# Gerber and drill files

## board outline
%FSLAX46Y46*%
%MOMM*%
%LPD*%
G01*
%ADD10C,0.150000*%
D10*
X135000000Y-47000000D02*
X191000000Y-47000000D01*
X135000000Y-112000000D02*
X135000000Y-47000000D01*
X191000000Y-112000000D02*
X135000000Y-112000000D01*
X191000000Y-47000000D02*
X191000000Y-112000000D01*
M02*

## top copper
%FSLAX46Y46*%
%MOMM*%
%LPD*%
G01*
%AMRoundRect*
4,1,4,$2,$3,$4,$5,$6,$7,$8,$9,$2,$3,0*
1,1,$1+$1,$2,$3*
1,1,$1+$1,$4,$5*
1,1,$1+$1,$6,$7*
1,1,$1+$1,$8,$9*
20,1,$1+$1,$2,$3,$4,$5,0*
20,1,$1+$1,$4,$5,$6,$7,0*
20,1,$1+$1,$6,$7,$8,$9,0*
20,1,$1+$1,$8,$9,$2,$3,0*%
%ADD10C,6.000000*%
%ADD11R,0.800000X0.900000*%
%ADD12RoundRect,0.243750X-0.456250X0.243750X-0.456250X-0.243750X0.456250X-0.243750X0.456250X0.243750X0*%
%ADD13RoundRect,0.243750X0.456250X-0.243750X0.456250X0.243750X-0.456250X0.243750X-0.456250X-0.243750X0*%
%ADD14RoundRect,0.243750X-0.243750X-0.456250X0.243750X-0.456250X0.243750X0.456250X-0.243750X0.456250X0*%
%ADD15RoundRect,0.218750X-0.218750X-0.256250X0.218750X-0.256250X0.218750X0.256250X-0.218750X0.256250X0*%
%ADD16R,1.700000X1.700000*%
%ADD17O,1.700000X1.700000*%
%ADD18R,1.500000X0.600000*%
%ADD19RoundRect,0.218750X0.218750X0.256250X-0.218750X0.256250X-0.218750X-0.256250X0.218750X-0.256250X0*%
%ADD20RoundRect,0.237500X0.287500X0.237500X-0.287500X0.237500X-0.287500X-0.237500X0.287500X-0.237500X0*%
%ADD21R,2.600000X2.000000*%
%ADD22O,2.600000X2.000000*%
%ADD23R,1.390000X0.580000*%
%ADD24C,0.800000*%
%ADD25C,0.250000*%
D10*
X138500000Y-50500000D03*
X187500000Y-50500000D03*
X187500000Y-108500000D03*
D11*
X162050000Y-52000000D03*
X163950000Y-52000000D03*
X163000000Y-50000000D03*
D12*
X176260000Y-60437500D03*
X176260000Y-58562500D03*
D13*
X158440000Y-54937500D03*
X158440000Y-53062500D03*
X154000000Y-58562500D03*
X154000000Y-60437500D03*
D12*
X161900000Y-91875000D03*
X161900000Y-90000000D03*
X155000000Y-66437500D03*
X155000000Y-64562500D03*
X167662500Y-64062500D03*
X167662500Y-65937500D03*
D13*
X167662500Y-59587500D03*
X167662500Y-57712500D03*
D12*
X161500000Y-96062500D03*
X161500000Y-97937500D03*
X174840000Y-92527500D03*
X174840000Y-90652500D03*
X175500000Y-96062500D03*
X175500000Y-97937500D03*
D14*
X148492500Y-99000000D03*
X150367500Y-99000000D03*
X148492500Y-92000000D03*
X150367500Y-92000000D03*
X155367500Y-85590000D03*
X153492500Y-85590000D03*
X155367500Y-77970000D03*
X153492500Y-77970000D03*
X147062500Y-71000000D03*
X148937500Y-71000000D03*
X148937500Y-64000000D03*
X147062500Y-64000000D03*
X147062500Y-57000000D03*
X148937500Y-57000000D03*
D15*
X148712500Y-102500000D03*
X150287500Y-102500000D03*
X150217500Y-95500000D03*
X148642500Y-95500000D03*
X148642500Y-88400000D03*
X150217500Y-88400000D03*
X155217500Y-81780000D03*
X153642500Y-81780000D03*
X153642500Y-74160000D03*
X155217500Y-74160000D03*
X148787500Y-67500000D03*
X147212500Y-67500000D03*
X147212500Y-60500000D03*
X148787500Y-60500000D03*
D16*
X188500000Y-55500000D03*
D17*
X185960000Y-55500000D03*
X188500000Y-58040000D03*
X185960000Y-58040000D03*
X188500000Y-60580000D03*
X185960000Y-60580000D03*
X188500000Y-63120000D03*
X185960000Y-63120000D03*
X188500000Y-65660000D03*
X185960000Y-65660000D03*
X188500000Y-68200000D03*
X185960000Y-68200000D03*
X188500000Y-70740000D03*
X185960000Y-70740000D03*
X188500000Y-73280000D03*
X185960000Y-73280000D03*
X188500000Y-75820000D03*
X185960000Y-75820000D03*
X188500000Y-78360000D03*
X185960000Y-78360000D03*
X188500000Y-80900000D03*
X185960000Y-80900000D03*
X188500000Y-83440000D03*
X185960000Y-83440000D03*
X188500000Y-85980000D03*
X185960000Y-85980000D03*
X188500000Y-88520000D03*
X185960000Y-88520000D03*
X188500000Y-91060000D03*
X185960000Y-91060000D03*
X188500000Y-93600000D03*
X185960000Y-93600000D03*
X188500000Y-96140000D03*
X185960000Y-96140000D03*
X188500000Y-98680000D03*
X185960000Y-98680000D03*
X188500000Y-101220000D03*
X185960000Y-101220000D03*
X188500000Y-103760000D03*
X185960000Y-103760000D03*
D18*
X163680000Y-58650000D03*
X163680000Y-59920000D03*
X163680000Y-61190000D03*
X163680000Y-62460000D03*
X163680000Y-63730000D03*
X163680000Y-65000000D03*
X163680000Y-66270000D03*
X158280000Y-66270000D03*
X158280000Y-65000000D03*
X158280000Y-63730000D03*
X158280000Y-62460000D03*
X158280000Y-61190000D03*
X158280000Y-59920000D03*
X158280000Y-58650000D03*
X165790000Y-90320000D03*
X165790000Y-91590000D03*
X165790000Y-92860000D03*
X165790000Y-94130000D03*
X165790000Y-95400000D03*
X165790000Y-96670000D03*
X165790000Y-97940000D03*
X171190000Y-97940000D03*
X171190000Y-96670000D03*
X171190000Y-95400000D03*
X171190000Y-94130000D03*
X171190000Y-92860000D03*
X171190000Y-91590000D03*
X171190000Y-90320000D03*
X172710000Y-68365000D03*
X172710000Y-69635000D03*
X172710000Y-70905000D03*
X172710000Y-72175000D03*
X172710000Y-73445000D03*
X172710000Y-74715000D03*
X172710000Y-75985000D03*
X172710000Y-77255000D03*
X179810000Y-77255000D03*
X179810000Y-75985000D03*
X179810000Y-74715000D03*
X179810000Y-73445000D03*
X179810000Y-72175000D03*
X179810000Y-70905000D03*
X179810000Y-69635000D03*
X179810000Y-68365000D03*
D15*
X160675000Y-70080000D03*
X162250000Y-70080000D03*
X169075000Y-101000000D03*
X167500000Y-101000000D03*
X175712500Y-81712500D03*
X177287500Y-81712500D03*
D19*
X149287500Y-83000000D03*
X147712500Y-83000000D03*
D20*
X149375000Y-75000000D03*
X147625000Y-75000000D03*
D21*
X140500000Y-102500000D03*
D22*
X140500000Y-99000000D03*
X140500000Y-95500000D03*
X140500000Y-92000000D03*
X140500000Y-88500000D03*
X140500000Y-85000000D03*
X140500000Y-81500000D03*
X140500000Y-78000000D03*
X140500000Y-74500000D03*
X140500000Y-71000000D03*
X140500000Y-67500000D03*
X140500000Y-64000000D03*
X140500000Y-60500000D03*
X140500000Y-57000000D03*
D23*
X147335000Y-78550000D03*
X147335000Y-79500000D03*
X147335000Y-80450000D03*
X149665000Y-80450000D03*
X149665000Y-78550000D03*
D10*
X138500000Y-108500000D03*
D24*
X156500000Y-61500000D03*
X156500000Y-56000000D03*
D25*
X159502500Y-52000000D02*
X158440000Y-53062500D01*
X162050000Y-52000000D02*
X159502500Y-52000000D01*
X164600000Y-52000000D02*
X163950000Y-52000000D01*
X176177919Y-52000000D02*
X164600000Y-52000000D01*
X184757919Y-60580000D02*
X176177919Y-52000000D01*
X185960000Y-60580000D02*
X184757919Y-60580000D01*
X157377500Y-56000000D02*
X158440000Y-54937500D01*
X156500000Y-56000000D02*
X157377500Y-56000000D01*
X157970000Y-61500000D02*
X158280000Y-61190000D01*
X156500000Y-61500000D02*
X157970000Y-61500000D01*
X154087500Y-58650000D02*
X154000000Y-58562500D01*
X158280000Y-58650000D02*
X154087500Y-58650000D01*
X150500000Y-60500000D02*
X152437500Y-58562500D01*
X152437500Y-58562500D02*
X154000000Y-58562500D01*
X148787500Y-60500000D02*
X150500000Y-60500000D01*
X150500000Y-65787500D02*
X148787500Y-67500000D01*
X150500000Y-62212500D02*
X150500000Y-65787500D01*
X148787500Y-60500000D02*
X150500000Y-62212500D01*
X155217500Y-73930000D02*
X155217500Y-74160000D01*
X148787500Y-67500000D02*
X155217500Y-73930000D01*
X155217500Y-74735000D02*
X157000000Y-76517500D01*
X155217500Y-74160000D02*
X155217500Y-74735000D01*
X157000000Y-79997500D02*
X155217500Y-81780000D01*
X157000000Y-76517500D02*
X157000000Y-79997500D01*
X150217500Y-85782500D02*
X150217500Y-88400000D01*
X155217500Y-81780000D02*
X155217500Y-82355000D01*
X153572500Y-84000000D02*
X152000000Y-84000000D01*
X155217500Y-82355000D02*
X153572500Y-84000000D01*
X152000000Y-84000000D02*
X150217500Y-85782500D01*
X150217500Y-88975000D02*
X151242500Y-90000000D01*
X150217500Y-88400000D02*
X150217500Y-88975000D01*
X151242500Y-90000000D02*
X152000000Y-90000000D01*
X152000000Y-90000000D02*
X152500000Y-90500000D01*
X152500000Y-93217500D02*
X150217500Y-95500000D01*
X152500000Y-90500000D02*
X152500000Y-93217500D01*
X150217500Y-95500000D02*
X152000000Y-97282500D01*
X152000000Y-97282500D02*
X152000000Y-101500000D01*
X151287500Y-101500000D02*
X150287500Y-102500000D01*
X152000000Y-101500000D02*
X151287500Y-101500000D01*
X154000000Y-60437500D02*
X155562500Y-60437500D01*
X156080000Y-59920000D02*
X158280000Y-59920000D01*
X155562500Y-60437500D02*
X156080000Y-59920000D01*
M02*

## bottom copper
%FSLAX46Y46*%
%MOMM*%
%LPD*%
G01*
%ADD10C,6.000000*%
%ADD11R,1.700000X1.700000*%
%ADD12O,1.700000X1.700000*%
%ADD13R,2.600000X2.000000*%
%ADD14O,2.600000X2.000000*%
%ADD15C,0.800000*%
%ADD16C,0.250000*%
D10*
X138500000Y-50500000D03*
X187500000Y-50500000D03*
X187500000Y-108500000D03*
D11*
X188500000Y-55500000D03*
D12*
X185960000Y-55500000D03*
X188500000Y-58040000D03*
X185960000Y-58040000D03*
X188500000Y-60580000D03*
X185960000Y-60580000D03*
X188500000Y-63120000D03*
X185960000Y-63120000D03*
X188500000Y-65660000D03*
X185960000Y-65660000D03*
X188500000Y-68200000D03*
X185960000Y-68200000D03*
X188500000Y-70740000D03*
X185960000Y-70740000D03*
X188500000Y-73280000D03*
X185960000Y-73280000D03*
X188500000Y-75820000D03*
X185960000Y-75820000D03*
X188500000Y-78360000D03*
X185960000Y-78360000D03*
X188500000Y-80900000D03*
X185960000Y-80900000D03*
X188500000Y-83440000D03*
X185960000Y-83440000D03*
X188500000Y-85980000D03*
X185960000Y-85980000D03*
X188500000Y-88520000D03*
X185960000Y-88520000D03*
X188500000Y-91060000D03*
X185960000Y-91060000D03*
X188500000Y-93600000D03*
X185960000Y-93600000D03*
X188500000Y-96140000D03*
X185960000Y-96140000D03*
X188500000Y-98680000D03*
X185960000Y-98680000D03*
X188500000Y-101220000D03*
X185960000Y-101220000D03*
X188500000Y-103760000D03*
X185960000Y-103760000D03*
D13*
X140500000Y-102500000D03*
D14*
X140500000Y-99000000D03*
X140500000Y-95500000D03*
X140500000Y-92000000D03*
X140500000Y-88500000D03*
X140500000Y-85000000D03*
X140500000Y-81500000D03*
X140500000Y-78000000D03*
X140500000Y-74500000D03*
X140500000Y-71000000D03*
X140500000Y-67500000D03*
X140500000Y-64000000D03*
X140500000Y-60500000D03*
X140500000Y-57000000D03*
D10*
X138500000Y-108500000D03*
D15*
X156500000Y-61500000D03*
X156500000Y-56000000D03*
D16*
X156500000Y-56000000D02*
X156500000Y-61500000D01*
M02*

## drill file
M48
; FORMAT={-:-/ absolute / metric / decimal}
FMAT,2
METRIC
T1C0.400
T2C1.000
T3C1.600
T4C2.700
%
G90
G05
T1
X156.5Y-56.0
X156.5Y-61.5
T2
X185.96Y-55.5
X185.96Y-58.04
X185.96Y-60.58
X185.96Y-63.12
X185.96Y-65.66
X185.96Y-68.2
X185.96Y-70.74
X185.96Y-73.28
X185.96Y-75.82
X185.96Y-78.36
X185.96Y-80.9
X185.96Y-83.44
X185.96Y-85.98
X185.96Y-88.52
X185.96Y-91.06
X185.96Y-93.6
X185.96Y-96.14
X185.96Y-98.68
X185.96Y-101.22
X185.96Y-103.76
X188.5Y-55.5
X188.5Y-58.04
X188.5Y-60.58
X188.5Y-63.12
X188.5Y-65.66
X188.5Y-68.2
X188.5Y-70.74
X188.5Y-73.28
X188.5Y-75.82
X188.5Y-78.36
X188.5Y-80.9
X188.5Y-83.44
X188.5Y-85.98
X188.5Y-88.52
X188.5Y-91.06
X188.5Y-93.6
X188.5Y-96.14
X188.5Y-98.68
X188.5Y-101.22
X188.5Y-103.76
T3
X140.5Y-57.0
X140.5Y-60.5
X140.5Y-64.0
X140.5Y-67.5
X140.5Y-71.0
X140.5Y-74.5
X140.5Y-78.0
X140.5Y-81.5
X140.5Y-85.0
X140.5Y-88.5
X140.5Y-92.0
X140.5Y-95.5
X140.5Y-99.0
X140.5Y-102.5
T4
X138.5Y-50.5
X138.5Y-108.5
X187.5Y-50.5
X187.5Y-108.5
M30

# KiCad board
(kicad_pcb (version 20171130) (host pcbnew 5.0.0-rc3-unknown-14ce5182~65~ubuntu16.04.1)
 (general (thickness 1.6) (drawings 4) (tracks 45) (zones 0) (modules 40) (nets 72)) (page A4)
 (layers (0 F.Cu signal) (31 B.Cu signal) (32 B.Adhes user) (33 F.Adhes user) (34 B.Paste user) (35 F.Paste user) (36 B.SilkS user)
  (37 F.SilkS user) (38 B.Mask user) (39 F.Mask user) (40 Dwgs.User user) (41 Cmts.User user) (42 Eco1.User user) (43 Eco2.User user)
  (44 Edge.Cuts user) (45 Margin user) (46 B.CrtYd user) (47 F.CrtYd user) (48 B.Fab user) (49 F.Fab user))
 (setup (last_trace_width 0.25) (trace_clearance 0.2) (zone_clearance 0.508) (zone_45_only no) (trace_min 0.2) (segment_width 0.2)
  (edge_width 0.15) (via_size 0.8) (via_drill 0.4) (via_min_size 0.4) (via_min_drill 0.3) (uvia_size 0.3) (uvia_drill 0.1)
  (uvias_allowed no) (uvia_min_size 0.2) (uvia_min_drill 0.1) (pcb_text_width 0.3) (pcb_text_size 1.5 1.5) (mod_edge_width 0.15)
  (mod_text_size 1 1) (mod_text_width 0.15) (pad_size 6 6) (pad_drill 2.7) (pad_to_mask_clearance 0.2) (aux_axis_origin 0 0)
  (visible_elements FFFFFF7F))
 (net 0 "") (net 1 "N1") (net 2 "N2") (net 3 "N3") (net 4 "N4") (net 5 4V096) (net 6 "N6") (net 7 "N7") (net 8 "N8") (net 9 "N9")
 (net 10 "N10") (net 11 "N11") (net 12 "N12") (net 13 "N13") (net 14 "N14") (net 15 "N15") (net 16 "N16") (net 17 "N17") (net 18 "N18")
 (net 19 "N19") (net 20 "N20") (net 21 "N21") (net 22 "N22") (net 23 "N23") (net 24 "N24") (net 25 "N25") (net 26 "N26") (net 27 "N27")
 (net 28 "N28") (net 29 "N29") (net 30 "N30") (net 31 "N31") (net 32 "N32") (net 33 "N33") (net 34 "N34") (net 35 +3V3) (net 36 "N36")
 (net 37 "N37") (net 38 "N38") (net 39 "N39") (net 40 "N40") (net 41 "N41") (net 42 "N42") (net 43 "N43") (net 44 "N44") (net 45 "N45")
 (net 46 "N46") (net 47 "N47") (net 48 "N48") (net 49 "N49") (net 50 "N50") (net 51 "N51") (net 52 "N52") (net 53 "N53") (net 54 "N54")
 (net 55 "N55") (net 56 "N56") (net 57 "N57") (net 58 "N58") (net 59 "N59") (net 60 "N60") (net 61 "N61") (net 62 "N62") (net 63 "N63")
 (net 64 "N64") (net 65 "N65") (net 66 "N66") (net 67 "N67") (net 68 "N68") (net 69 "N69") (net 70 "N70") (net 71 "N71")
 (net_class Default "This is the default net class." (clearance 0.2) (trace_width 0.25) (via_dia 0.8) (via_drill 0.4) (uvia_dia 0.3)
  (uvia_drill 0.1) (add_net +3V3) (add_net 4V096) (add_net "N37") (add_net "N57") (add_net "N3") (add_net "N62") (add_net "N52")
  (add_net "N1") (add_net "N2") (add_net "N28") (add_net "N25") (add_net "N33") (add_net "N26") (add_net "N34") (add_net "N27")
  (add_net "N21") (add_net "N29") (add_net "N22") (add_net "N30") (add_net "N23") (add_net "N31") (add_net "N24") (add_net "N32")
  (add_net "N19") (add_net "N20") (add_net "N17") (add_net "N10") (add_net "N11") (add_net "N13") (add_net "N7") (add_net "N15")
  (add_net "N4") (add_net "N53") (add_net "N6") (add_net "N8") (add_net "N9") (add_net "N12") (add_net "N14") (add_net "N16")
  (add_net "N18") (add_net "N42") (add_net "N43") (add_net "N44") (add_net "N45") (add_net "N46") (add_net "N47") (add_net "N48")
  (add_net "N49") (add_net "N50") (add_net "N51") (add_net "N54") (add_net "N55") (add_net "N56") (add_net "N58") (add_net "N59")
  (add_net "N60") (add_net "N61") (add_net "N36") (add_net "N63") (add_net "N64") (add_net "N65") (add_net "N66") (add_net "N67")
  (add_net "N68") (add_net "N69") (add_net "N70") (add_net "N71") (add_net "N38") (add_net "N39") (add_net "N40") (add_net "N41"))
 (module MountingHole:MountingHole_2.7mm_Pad (layer F.Cu) (at 138.5 50.5 180)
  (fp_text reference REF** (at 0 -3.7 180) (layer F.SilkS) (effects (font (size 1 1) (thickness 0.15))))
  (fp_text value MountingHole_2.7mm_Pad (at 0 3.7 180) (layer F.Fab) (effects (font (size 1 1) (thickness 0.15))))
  (pad 1 thru_hole circle (at 0 0 180) (size 6 6) (drill 2.7) (layers *.Cu *.Mask)))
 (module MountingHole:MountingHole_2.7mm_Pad (layer F.Cu) (at 187.5 50.5 180)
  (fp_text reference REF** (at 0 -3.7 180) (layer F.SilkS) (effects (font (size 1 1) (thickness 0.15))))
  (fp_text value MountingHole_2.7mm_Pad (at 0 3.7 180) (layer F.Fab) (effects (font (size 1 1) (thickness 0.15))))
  (pad 1 thru_hole circle (at 0 0 180) (size 6 6) (drill 2.7) (layers *.Cu *.Mask)))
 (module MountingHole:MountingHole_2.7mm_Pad (layer F.Cu) (at 187.5 108.5 180)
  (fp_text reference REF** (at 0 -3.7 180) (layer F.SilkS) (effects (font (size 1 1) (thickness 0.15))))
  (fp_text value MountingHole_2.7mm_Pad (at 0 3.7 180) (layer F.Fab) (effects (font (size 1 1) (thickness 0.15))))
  (pad 1 thru_hole circle (at 0 0 180) (size 6 6) (drill 2.7) (layers *.Cu *.Mask)))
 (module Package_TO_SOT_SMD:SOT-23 (layer F.Cu) (at 163 51 90)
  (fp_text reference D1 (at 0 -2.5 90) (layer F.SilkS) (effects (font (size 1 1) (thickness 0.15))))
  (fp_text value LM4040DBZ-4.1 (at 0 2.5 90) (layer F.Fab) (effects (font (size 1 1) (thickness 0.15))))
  (pad 1 smd rect (at -1 -0.95 90) (size 0.9 0.8) (layers F.Cu F.Paste F.Mask) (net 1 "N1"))
  (pad 2 smd rect (at -1 0.95 90) (size 0.9 0.8) (layers F.Cu F.Paste F.Mask) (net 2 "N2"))
  (pad 3 smd rect (at 1 0 90) (size 0.9 0.8) (layers F.Cu F.Paste F.Mask)))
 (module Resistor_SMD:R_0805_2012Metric (layer F.Cu) (at 176.26 59.5 270)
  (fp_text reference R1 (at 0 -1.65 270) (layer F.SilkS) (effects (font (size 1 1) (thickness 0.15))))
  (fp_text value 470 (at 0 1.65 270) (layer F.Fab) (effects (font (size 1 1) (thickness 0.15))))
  (pad 2 smd roundrect (at 0.9375 0 270) (size 0.975 1.4) (layers F.Cu F.Paste F.Mask) (roundrect_rratio 0.25) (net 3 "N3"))
  (pad 1 smd roundrect (at -0.9375 0 270) (size 0.975 1.4) (layers F.Cu F.Paste F.Mask) (roundrect_rratio 0.25) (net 1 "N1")))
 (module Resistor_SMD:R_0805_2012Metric (layer F.Cu) (at 158.44 54 90)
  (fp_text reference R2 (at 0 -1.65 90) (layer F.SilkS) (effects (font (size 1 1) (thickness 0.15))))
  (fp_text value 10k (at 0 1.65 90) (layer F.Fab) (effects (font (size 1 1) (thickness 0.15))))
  (pad 1 smd roundrect (at -0.9375 0 90) (size 0.975 1.4) (layers F.Cu F.Paste F.Mask) (roundrect_rratio 0.25) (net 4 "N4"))
  (pad 2 smd roundrect (at 0.9375 0 90) (size 0.975 1.4) (layers F.Cu F.Paste F.Mask) (roundrect_rratio 0.25) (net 1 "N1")))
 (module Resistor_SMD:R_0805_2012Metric (layer F.Cu) (at 154 59.5 90)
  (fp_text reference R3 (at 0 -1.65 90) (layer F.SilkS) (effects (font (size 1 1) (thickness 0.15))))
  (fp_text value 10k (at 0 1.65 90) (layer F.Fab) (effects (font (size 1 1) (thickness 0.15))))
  (pad 2 smd roundrect (at 0.9375 0 90) (size 0.975 1.4) (layers F.Cu F.Paste F.Mask) (roundrect_rratio 0.25) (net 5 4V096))
  (pad 1 smd roundrect (at -0.9375 0 90) (size 0.975 1.4) (layers F.Cu F.Paste F.Mask) (roundrect_rratio 0.25) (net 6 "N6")))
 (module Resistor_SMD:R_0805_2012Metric (layer F.Cu) (at 161.9 90.9375 270)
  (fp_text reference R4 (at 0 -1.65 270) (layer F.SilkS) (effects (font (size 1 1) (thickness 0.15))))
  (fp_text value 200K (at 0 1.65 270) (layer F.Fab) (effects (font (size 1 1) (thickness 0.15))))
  (pad 2 smd roundrect (at 0.9375 0 270) (size 0.975 1.4) (layers F.Cu F.Paste F.Mask) (roundrect_rratio 0.25) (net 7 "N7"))
  (pad 1 smd roundrect (at -0.9375 0 270) (size 0.975 1.4) (layers F.Cu F.Paste F.Mask) (roundrect_rratio 0.25) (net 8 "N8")))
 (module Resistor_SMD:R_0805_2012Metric (layer F.Cu) (at 155 65.5 270)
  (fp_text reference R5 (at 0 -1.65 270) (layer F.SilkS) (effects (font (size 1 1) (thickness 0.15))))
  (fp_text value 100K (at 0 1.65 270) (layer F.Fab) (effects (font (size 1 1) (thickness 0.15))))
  (pad 2 smd roundrect (at 0.9375 0 270) (size 0.975 1.4) (layers F.Cu F.Paste F.Mask) (roundrect_rratio 0.25) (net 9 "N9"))
  (pad 1 smd roundrect (at -0.9375 0 270) (size 0.975 1.4) (layers F.Cu F.Paste F.Mask) (roundrect_rratio 0.25) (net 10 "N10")))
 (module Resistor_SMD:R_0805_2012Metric (layer F.Cu) (at 167.6625 65 270)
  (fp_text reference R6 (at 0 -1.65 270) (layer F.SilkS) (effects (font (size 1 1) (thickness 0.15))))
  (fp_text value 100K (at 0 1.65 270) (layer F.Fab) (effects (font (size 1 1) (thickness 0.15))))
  (pad 1 smd roundrect (at -0.9375 0 270) (size 0.975 1.4) (layers F.Cu F.Paste F.Mask) (roundrect_rratio 0.25) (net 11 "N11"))
  (pad 2 smd roundrect (at 0.9375 0 270) (size 0.975 1.4) (layers F.Cu F.Paste F.Mask) (roundrect_rratio 0.25) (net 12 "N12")))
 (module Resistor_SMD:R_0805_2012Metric (layer F.Cu) (at 167.6625 58.65 90)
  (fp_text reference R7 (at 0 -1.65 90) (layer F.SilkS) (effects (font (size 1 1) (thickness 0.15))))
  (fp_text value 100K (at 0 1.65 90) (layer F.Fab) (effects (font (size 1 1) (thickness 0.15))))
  (pad 1 smd roundrect (at -0.9375 0 90) (size 0.975 1.4) (layers F.Cu F.Paste F.Mask) (roundrect_rratio 0.25) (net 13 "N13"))
  (pad 2 smd roundrect (at 0.9375 0 90) (size 0.975 1.4) (layers F.Cu F.Paste F.Mask) (roundrect_rratio 0.25) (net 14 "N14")))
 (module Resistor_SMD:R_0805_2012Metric (layer F.Cu) (at 161.5 97 270)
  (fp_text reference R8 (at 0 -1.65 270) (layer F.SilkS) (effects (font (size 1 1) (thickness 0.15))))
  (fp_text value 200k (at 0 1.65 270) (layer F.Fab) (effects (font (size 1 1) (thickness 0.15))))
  (pad 1 smd roundrect (at -0.9375 0 270) (size 0.975 1.4) (layers F.Cu F.Paste F.Mask) (roundrect_rratio 0.25) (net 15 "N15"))
  (pad 2 smd roundrect (at 0.9375 0 270) (size 0.975 1.4) (layers F.Cu F.Paste F.Mask) (roundrect_rratio 0.25) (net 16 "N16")))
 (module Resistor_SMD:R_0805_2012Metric (layer F.Cu) (at 174.84 91.59 270)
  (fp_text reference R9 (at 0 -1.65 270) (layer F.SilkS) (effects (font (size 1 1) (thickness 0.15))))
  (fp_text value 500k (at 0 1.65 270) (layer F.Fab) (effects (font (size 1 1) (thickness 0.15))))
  (pad 2 smd roundrect (at 0.9375 0 270) (size 0.975 1.4) (layers F.Cu F.Paste F.Mask) (roundrect_rratio 0.25) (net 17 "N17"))
  (pad 1 smd roundrect (at -0.9375 0 270) (size 0.975 1.4) (layers F.Cu F.Paste F.Mask) (roundrect_rratio 0.25) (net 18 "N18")))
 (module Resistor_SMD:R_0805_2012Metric (layer F.Cu) (at 175.5 97 270)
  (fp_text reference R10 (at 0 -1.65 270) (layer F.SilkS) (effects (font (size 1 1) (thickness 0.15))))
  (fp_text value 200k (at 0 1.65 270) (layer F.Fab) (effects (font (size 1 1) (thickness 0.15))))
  (pad 1 smd roundrect (at -0.9375 0 270) (size 0.975 1.4) (layers F.Cu F.Paste F.Mask) (roundrect_rratio 0.25) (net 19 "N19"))
  (pad 2 smd roundrect (at 0.9375 0 270) (size 0.975 1.4) (layers F.Cu F.Paste F.Mask) (roundrect_rratio 0.25) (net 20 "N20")))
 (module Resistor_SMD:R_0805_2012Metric (layer F.Cu) (at 149.43 99)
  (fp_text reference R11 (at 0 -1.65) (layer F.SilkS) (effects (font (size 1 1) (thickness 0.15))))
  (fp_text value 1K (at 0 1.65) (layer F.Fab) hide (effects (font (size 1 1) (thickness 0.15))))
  (pad 1 smd roundrect (at -0.9375 0) (size 0.975 1.4) (layers F.Cu F.Paste F.Mask) (roundrect_rratio 0.25) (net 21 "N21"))
  (pad 2 smd roundrect (at 0.9375 0) (size 0.975 1.4) (layers F.Cu F.Paste F.Mask) (roundrect_rratio 0.25) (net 17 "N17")))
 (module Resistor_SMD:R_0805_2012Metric (layer F.Cu) (at 149.43 92)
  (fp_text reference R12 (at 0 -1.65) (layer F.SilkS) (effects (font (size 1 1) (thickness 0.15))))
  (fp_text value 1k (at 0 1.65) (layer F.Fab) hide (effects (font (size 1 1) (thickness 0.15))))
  (pad 1 smd roundrect (at -0.9375 0) (size 0.975 1.4) (layers F.Cu F.Paste F.Mask) (roundrect_rratio 0.25) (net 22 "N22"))
  (pad 2 smd roundrect (at 0.9375 0) (size 0.975 1.4) (layers F.Cu F.Paste F.Mask) (roundrect_rratio 0.25) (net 10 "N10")))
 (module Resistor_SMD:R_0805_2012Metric (layer F.Cu) (at 154.43 85.59)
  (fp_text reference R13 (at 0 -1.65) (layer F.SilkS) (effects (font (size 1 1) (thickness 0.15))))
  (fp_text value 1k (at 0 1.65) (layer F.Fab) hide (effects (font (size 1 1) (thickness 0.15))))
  (pad 2 smd roundrect (at 0.9375 0) (size 0.975 1.4) (layers F.Cu F.Paste F.Mask) (roundrect_rratio 0.25) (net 11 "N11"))
  (pad 1 smd roundrect (at -0.9375 0) (size 0.975 1.4) (layers F.Cu F.Paste F.Mask) (roundrect_rratio 0.25) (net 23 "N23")))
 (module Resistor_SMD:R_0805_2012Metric (layer F.Cu) (at 154.43 77.97)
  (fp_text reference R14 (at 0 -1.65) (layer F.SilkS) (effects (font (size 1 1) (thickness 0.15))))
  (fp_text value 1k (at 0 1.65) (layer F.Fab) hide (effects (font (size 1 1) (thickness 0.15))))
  (pad 2 smd roundrect (at 0.9375 0) (size 0.975 1.4) (layers F.Cu F.Paste F.Mask) (roundrect_rratio 0.25) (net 13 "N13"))
  (pad 1 smd roundrect (at -0.9375 0) (size 0.975 1.4) (layers F.Cu F.Paste F.Mask) (roundrect_rratio 0.25) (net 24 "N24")))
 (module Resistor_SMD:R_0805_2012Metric (layer F.Cu) (at 148 71)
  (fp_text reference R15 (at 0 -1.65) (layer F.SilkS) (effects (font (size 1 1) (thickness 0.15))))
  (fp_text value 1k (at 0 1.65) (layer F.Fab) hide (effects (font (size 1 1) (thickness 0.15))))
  (pad 1 smd roundrect (at -0.9375 0) (size 0.975 1.4) (layers F.Cu F.Paste F.Mask) (roundrect_rratio 0.25) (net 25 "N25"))
  (pad 2 smd roundrect (at 0.9375 0) (size 0.975 1.4) (layers F.Cu F.Paste F.Mask) (roundrect_rratio 0.25) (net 7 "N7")))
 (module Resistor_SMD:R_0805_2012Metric (layer F.Cu) (at 148 64)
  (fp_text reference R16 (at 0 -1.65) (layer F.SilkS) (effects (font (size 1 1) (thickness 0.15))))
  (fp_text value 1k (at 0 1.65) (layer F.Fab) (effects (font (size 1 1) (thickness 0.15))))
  (pad 2 smd roundrect (at 0.9375 0) (size 0.975 1.4) (layers F.Cu F.Paste F.Mask) (roundrect_rratio 0.25) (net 15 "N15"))
  (pad 1 smd roundrect (at -0.9375 0) (size 0.975 1.4) (layers F.Cu F.Paste F.Mask) (roundrect_rratio 0.25) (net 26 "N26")))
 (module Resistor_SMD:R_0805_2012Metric (layer F.Cu) (at 148 57)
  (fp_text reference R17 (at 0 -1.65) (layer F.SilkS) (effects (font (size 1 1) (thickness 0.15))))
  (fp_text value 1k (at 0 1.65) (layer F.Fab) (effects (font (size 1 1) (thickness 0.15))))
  (pad 1 smd roundrect (at -0.9375 0) (size 0.975 1.4) (layers F.Cu F.Paste F.Mask) (roundrect_rratio 0.25) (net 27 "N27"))
  (pad 2 smd roundrect (at 0.9375 0) (size 0.975 1.4) (layers F.Cu F.Paste F.Mask) (roundrect_rratio 0.25) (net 19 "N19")))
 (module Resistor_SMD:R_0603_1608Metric (layer F.Cu) (at 149.5 102.5)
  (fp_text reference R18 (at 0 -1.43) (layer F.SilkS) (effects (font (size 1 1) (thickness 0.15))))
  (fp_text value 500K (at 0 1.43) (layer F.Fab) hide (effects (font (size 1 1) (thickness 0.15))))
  (pad 1 smd roundrect (at -0.7875 0) (size 0.875 0.95) (layers F.Cu F.Paste F.Mask) (roundrect_rratio 0.25) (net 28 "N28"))
  (pad 2 smd roundrect (at 0.7875 0) (size 0.875 0.95) (layers F.Cu F.Paste F.Mask) (roundrect_rratio 0.25) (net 5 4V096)))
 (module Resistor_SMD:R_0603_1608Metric (layer F.Cu) (at 149.43 95.5)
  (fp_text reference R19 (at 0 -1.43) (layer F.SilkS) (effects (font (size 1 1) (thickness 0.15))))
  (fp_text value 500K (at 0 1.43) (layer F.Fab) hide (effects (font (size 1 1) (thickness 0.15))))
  (pad 2 smd roundrect (at 0.7875 0) (size 0.875 0.95) (layers F.Cu F.Paste F.Mask) (roundrect_rratio 0.25) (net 5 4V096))
  (pad 1 smd roundrect (at -0.7875 0) (size 0.875 0.95) (layers F.Cu F.Paste F.Mask) (roundrect_rratio 0.25) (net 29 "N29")))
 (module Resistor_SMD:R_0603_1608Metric (layer F.Cu) (at 149.43 88.4)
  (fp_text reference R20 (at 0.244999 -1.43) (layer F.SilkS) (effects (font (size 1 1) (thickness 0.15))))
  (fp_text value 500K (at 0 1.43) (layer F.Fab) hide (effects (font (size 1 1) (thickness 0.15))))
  (pad 1 smd roundrect (at -0.7875 0) (size 0.875 0.95) (layers F.Cu F.Paste F.Mask) (roundrect_rratio 0.25) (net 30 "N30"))
  (pad 2 smd roundrect (at 0.7875 0) (size 0.875 0.95) (layers F.Cu F.Paste F.Mask) (roundrect_rratio 0.25) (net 5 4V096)))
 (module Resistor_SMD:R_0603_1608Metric (layer F.Cu) (at 154.43 81.78)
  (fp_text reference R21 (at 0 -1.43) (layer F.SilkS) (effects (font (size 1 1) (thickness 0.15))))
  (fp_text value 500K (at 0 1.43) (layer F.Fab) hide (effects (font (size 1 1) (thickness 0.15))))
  (pad 2 smd roundrect (at 0.7875 0) (size 0.875 0.95) (layers F.Cu F.Paste F.Mask) (roundrect_rratio 0.25) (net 5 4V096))
  (pad 1 smd roundrect (at -0.7875 0) (size 0.875 0.95) (layers F.Cu F.Paste F.Mask) (roundrect_rratio 0.25) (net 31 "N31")))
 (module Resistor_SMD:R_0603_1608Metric (layer F.Cu) (at 154.43 74.16)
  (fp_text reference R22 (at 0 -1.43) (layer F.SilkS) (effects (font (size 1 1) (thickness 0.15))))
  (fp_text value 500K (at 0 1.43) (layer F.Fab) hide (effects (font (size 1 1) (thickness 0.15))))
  (pad 1 smd roundrect (at -0.7875 0) (size 0.875 0.95) (layers F.Cu F.Paste F.Mask) (roundrect_rratio 0.25) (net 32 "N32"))
  (pad 2 smd roundrect (at 0.7875 0) (size 0.875 0.95) (layers F.Cu F.Paste F.Mask) (roundrect_rratio 0.25) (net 5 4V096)))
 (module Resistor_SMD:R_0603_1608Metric (layer F.Cu) (at 148 67.5)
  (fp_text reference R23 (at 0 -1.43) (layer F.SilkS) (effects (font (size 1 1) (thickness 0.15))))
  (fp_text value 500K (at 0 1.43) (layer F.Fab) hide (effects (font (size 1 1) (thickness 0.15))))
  (pad 2 smd roundrect (at 0.7875 0) (size 0.875 0.95) (layers F.Cu F.Paste F.Mask) (roundrect_rratio 0.25) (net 5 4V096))
  (pad 1 smd roundrect (at -0.7875 0) (size 0.875 0.95) (layers F.Cu F.Paste F.Mask) (roundrect_rratio 0.25) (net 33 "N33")))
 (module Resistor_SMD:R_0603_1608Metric (layer F.Cu) (at 148 60.5)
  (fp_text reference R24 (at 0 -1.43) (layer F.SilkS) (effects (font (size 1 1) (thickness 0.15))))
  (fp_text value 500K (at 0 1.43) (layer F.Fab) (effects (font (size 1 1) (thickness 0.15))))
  (pad 1 smd roundrect (at -0.7875 0) (size 0.875 0.95) (layers F.Cu F.Paste F.Mask) (roundrect_rratio 0.25) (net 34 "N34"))
  (pad 2 smd roundrect (at 0.7875 0) (size 0.875 0.95) (layers F.Cu F.Paste F.Mask) (roundrect_rratio 0.25) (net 5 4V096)))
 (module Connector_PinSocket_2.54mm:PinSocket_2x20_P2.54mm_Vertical (layer F.Cu) (at 188.5 55.5)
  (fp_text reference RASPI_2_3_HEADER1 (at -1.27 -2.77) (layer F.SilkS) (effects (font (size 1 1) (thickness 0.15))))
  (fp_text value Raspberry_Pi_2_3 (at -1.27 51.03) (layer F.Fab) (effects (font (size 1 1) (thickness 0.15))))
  (pad 1 thru_hole rect (at 0 0) (size 1.7 1.7) (drill 1) (layers *.Cu *.Mask) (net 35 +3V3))
  (pad 2 thru_hole oval (at -2.54 0) (size 1.7 1.7) (drill 1) (layers *.Cu *.Mask) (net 3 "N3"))
  (pad 3 thru_hole oval (at 0 2.54) (size 1.7 1.7) (drill 1) (layers *.Cu *.Mask) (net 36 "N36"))
  (pad 4 thru_hole oval (at -2.54 2.54) (size 1.7 1.7) (drill 1) (layers *.Cu *.Mask) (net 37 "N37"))
  (pad 5 thru_hole oval (at 0 5.08) (size 1.7 1.7) (drill 1) (layers *.Cu *.Mask) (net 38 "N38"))
  (pad 6 thru_hole oval (at -2.54 5.08) (size 1.7 1.7) (drill 1) (layers *.Cu *.Mask) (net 2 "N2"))
  (pad 7 thru_hole oval (at 0 7.62) (size 1.7 1.7) (drill 1) (layers *.Cu *.Mask) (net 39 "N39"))
  (pad 8 thru_hole oval (at -2.54 7.62) (size 1.7 1.7) (drill 1) (layers *.Cu *.Mask) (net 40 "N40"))
  (pad 9 thru_hole oval (at 0 10.16) (size 1.7 1.7) (drill 1) (layers *.Cu *.Mask) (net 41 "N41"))
  (pad 10 thru_hole oval (at -2.54 10.16) (size 1.7 1.7) (drill 1) (layers *.Cu *.Mask) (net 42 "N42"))
  (pad 11 thru_hole oval (at 0 12.7) (size 1.7 1.7) (drill 1) (layers *.Cu *.Mask) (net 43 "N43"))
  (pad 12 thru_hole oval (at -2.54 12.7) (size 1.7 1.7) (drill 1) (layers *.Cu *.Mask) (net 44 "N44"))
  (pad 13 thru_hole oval (at 0 15.24) (size 1.7 1.7) (drill 1) (layers *.Cu *.Mask) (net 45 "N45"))
  (pad 14 thru_hole oval (at -2.54 15.24) (size 1.7 1.7) (drill 1) (layers *.Cu *.Mask) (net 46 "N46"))
  (pad 15 thru_hole oval (at 0 17.78) (size 1.7 1.7) (drill 1) (layers *.Cu *.Mask) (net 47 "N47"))
  (pad 16 thru_hole oval (at -2.54 17.78) (size 1.7 1.7) (drill 1) (layers *.Cu *.Mask) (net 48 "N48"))
  (pad 17 thru_hole oval (at 0 20.32) (size 1.7 1.7) (drill 1) (layers *.Cu *.Mask) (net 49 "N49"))
  (pad 18 thru_hole oval (at -2.54 20.32) (size 1.7 1.7) (drill 1) (layers *.Cu *.Mask) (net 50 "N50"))
  (pad 19 thru_hole oval (at 0 22.86) (size 1.7 1.7) (drill 1) (layers *.Cu *.Mask) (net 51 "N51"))
  (pad 20 thru_hole oval (at -2.54 22.86) (size 1.7 1.7) (drill 1) (layers *.Cu *.Mask) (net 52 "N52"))
  (pad 21 thru_hole oval (at 0 25.4) (size 1.7 1.7) (drill 1) (layers *.Cu *.Mask) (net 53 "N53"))
  (pad 22 thru_hole oval (at -2.54 25.4) (size 1.7 1.7) (drill 1) (layers *.Cu *.Mask) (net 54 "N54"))
  (pad 23 thru_hole oval (at 0 27.94) (size 1.7 1.7) (drill 1) (layers *.Cu *.Mask) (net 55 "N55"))
  (pad 24 thru_hole oval (at -2.54 27.94) (size 1.7 1.7) (drill 1) (layers *.Cu *.Mask) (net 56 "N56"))
  (pad 25 thru_hole oval (at 0 30.48) (size 1.7 1.7) (drill 1) (layers *.Cu *.Mask) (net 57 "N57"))
  (pad 26 thru_hole oval (at -2.54 30.48) (size 1.7 1.7) (drill 1) (layers *.Cu *.Mask) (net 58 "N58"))
  (pad 27 thru_hole oval (at 0 33.02) (size 1.7 1.7) (drill 1) (layers *.Cu *.Mask) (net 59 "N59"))
  (pad 28 thru_hole oval (at -2.54 33.02) (size 1.7 1.7) (drill 1) (layers *.Cu *.Mask) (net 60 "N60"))
  (pad 29 thru_hole oval (at 0 35.56) (size 1.7 1.7) (drill 1) (layers *.Cu *.Mask) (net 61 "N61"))
  (pad 30 thru_hole oval (at -2.54 35.56) (size 1.7 1.7) (drill 1) (layers *.Cu *.Mask) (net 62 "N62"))
  (pad 31 thru_hole oval (at 0 38.1) (size 1.7 1.7) (drill 1) (layers *.Cu *.Mask) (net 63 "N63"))
  (pad 32 thru_hole oval (at -2.54 38.1) (size 1.7 1.7) (drill 1) (layers *.Cu *.Mask) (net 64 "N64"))
  (pad 33 thru_hole oval (at 0 40.64) (size 1.7 1.7) (drill 1) (layers *.Cu *.Mask) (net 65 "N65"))
  (pad 34 thru_hole oval (at -2.54 40.64) (size 1.7 1.7) (drill 1) (layers *.Cu *.Mask) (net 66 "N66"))
  (pad 35 thru_hole oval (at 0 43.18) (size 1.7 1.7) (drill 1) (layers *.Cu *.Mask) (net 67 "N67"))
  (pad 36 thru_hole oval (at -2.54 43.18) (size 1.7 1.7) (drill 1) (layers *.Cu *.Mask) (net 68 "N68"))
  (pad 37 thru_hole oval (at 0 45.72) (size 1.7 1.7) (drill 1) (layers *.Cu *.Mask) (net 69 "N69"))
  (pad 38 thru_hole oval (at -2.54 45.72) (size 1.7 1.7) (drill 1) (layers *.Cu *.Mask) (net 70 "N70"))
  (pad 39 thru_hole oval (at 0 48.26) (size 1.7 1.7) (drill 1) (layers *.Cu *.Mask) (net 37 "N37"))
  (pad 40 thru_hole oval (at -2.54 48.26) (size 1.7 1.7) (drill 1) (layers *.Cu *.Mask) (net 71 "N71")))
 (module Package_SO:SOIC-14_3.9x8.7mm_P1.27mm (layer F.Cu) (at 160.98 62.46)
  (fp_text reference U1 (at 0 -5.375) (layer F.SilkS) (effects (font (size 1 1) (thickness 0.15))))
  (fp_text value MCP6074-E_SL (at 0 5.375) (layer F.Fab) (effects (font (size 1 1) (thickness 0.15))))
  (pad 14 smd rect (at 2.7 -3.81) (size 1.5 0.6) (layers F.Cu F.Paste F.Mask) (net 14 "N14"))
  (pad 13 smd rect (at 2.7 -2.54) (size 1.5 0.6) (layers F.Cu F.Paste F.Mask) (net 13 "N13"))
  (pad 12 smd rect (at 2.7 -1.27) (size 1.5 0.6) (layers F.Cu F.Paste F.Mask) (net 5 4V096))
  (pad 11 smd rect (at 2.7 0) (size 1.5 0.6) (layers F.Cu F.Paste F.Mask) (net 57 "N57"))
  (pad 10 smd rect (at 2.7 1.27) (size 1.5 0.6) (layers F.Cu F.Paste F.Mask) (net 5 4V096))
  (pad 9 smd rect (at 2.7 2.54) (size 1.5 0.6) (layers F.Cu F.Paste F.Mask) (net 11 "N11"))
  (pad 8 smd rect (at 2.7 3.81) (size 1.5 0.6) (layers F.Cu F.Paste F.Mask) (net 12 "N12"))
  (pad 7 smd rect (at -2.7 3.81) (size 1.5 0.6) (layers F.Cu F.Paste F.Mask) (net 9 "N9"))
  (pad 6 smd rect (at -2.7 2.54) (size 1.5 0.6) (layers F.Cu F.Paste F.Mask) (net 10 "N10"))
  (pad 5 smd rect (at -2.7 1.27) (size 1.5 0.6) (layers F.Cu F.Paste F.Mask) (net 5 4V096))
  (pad 4 smd rect (at -2.7 0) (size 1.5 0.6) (layers F.Cu F.Paste F.Mask) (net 37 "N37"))
  (pad 3 smd rect (at -2.7 -1.27) (size 1.5 0.6) (layers F.Cu F.Paste F.Mask) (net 4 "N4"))
  (pad 2 smd rect (at -2.7 -2.54) (size 1.5 0.6) (layers F.Cu F.Paste F.Mask) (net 6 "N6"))
  (pad 1 smd rect (at -2.7 -3.81) (size 1.5 0.6) (layers F.Cu F.Paste F.Mask) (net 5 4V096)))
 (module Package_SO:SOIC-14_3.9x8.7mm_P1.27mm (layer F.Cu) (at 168.49 94.13)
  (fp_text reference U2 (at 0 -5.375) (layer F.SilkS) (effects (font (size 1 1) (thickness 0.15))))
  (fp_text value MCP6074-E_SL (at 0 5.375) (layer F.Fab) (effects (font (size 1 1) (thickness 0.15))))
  (pad 1 smd rect (at -2.7 -3.81) (size 1.5 0.6) (layers F.Cu F.Paste F.Mask) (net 8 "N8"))
  (pad 2 smd rect (at -2.7 -2.54) (size 1.5 0.6) (layers F.Cu F.Paste F.Mask) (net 7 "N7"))
  (pad 3 smd rect (at -2.7 -1.27) (size 1.5 0.6) (layers F.Cu F.Paste F.Mask) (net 5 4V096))
  (pad 4 smd rect (at -2.7 0) (size 1.5 0.6) (layers F.Cu F.Paste F.Mask) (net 37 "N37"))
  (pad 5 smd rect (at -2.7 1.27) (size 1.5 0.6) (layers F.Cu F.Paste F.Mask) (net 5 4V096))
  (pad 6 smd rect (at -2.7 2.54) (size 1.5 0.6) (layers F.Cu F.Paste F.Mask) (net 15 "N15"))
  (pad 7 smd rect (at -2.7 3.81) (size 1.5 0.6) (layers F.Cu F.Paste F.Mask) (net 16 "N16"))
  (pad 8 smd rect (at 2.7 3.81) (size 1.5 0.6) (layers F.Cu F.Paste F.Mask) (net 20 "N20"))
  (pad 9 smd rect (at 2.7 2.54) (size 1.5 0.6) (layers F.Cu F.Paste F.Mask) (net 19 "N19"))
  (pad 10 smd rect (at 2.7 1.27) (size 1.5 0.6) (layers F.Cu F.Paste F.Mask) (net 5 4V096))
  (pad 11 smd rect (at 2.7 0) (size 1.5 0.6) (layers F.Cu F.Paste F.Mask) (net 57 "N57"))
  (pad 12 smd rect (at 2.7 -1.27) (size 1.5 0.6) (layers F.Cu F.Paste F.Mask) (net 5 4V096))
  (pad 13 smd rect (at 2.7 -2.54) (size 1.5 0.6) (layers F.Cu F.Paste F.Mask) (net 17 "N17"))
  (pad 14 smd rect (at 2.7 -3.81) (size 1.5 0.6) (layers F.Cu F.Paste F.Mask) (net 18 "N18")))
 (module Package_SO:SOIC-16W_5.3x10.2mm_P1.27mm (layer F.Cu) (at 176.26 72.81)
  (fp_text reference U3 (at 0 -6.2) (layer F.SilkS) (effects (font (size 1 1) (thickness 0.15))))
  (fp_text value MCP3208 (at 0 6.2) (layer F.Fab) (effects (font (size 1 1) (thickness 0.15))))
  (pad 1 smd rect (at -3.55 -4.445) (size 1.5 0.6) (layers F.Cu F.Paste F.Mask) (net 5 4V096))
  (pad 2 smd rect (at -3.55 -3.175) (size 1.5 0.6) (layers F.Cu F.Paste F.Mask) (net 9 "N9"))
  (pad 3 smd rect (at -3.55 -1.905) (size 1.5 0.6) (layers F.Cu F.Paste F.Mask) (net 12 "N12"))
  (pad 4 smd rect (at -3.55 -0.635) (size 1.5 0.6) (layers F.Cu F.Paste F.Mask) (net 14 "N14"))
  (pad 5 smd rect (at -3.55 0.635) (size 1.5 0.6) (layers F.Cu F.Paste F.Mask) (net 8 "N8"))
  (pad 6 smd rect (at -3.55 1.905) (size 1.5 0.6) (layers F.Cu F.Paste F.Mask) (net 15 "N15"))
  (pad 7 smd rect (at -3.55 3.175) (size 1.5 0.6) (layers F.Cu F.Paste F.Mask) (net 19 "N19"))
  (pad 8 smd rect (at -3.55 4.445) (size 1.5 0.6) (layers F.Cu F.Paste F.Mask) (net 17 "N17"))
  (pad 9 smd rect (at 3.55 4.445) (size 1.5 0.6) (layers F.Cu F.Paste F.Mask) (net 62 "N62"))
  (pad 10 smd rect (at 3.55 3.175) (size 1.5 0.6) (layers F.Cu F.Paste F.Mask) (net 56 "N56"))
  (pad 11 smd rect (at 3.55 1.905) (size 1.5 0.6) (layers F.Cu F.Paste F.Mask) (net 51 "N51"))
  (pad 12 smd rect (at 3.55 0.635) (size 1.5 0.6) (layers F.Cu F.Paste F.Mask) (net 53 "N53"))
  (pad 13 smd rect (at 3.55 -0.635) (size 1.5 0.6) (layers F.Cu F.Paste F.Mask) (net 55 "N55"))
  (pad 14 smd rect (at 3.55 -1.905) (size 1.5 0.6) (layers F.Cu F.Paste F.Mask) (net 66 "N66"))
  (pad 15 smd rect (at 3.55 -3.175) (size 1.5 0.6) (layers F.Cu F.Paste F.Mask) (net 3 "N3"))
  (pad 16 smd rect (at 3.55 -4.445) (size 1.5 0.6) (layers F.Cu F.Paste F.Mask) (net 3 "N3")))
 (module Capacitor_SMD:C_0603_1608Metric (layer F.Cu) (at 161.4625 70.08)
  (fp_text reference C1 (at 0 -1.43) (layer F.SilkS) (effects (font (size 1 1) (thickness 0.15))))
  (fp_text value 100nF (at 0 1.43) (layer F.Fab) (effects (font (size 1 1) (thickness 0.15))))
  (pad 1 smd roundrect (at -0.7875 0) (size 0.875 0.95) (layers F.Cu F.Paste F.Mask) (roundrect_rratio 0.25) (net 37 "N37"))
  (pad 2 smd roundrect (at 0.7875 0) (size 0.875 0.95) (layers F.Cu F.Paste F.Mask) (roundrect_rratio 0.25) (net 57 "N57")))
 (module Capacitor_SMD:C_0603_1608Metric (layer F.Cu) (at 168.2875 101)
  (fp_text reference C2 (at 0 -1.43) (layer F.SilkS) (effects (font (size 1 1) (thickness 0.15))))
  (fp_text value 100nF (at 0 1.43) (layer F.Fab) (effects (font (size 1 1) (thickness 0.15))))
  (pad 2 smd roundrect (at 0.7875 0) (size 0.875 0.95) (layers F.Cu F.Paste F.Mask) (roundrect_rratio 0.25) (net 57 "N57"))
  (pad 1 smd roundrect (at -0.7875 0) (size 0.875 0.95) (layers F.Cu F.Paste F.Mask) (roundrect_rratio 0.25) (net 37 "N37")))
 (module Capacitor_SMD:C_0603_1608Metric (layer F.Cu) (at 176.5 81.7125)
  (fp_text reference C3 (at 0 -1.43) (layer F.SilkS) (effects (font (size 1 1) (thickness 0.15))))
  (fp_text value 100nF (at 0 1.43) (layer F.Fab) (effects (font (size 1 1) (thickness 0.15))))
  (pad 1 smd roundrect (at -0.7875 0) (size 0.875 0.95) (layers F.Cu F.Paste F.Mask) (roundrect_rratio 0.25) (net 3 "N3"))
  (pad 2 smd roundrect (at 0.7875 0) (size 0.875 0.95) (layers F.Cu F.Paste F.Mask) (roundrect_rratio 0.25) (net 62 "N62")))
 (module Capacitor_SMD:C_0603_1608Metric (layer F.Cu) (at 148.5 83 180)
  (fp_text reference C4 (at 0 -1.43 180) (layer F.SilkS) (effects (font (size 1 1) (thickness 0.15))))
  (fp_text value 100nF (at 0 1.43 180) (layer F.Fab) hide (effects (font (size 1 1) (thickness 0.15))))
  (pad 1 smd roundrect (at -0.7875 0 180) (size 0.875 0.95) (layers F.Cu F.Paste F.Mask) (roundrect_rratio 0.25) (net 3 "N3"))
  (pad 2 smd roundrect (at 0.7875 0 180) (size 0.875 0.95) (layers F.Cu F.Paste F.Mask) (roundrect_rratio 0.25) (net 52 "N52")))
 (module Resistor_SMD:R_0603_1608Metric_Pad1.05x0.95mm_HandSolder (layer F.Cu) (at 148.5 75 180)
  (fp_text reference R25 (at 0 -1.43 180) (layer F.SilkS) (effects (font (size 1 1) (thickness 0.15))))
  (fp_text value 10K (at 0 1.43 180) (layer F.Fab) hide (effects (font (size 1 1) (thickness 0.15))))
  (pad 1 smd roundrect (at -0.875 0 180) (size 1.05 0.95) (layers F.Cu F.Paste F.Mask) (roundrect_rratio 0.25) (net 53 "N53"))
  (pad 2 smd roundrect (at 0.875 0 180) (size 1.05 0.95) (layers F.Cu F.Paste F.Mask) (roundrect_rratio 0.25) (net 52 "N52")))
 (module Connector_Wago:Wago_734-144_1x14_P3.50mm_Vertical (layer F.Cu) (at 140.5 102.5 90)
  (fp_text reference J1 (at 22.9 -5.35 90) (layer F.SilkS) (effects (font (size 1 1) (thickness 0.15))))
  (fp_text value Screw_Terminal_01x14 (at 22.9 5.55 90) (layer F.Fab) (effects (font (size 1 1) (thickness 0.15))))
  (pad 1 thru_hole rect (at 0 0 90) (size 2 2.6) (drill 1.6) (layers *.Cu *.Mask) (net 28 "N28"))
  (pad 2 thru_hole oval (at 3.5 0 90) (size 2 2.6) (drill 1.6) (layers *.Cu *.Mask) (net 21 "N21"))
  (pad 3 thru_hole oval (at 7 0 90) (size 2 2.6) (drill 1.6) (layers *.Cu *.Mask) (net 29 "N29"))
  (pad 4 thru_hole oval (at 10.5 0 90) (size 2 2.6) (drill 1.6) (layers *.Cu *.Mask) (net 22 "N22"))
  (pad 5 thru_hole oval (at 14 0 90) (size 2 2.6) (drill 1.6) (layers *.Cu *.Mask) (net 30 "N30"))
  (pad 6 thru_hole oval (at 17.5 0 90) (size 2 2.6) (drill 1.6) (layers *.Cu *.Mask) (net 23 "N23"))
  (pad 7 thru_hole oval (at 21 0 90) (size 2 2.6) (drill 1.6) (layers *.Cu *.Mask) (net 31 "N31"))
  (pad 8 thru_hole oval (at 24.5 0 90) (size 2 2.6) (drill 1.6) (layers *.Cu *.Mask) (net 24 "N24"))
  (pad 9 thru_hole oval (at 28 0 90) (size 2 2.6) (drill 1.6) (layers *.Cu *.Mask) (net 32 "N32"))
  (pad 10 thru_hole oval (at 31.5 0 90) (size 2 2.6) (drill 1.6) (layers *.Cu *.Mask) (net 25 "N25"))
  (pad 11 thru_hole oval (at 35 0 90) (size 2 2.6) (drill 1.6) (layers *.Cu *.Mask) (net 33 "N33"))
  (pad 12 thru_hole oval (at 38.5 0 90) (size 2 2.6) (drill 1.6) (layers *.Cu *.Mask) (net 26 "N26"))
  (pad 13 thru_hole oval (at 42 0 90) (size 2 2.6) (drill 1.6) (layers *.Cu *.Mask) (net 34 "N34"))
  (pad 14 thru_hole oval (at 45.5 0 90) (size 2 2.6) (drill 1.6) (layers *.Cu *.Mask) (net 27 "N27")))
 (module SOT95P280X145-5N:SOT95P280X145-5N (layer F.Cu) (at 148.5 79.5)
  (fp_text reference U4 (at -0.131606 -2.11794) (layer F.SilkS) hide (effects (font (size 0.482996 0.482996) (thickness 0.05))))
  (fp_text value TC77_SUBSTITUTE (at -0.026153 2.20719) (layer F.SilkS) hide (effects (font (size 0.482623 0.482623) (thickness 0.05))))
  (pad 1 smd rect (at -1.165 -0.95 90) (size 0.58 1.39) (layers F.Cu F.Paste F.Mask) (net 58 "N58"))
  (pad 2 smd rect (at -1.165 0 90) (size 0.58 1.39) (layers F.Cu F.Paste F.Mask) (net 52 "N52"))
  (pad 3 smd rect (at -1.165 0.95 90) (size 0.58 1.39) (layers F.Cu F.Paste F.Mask) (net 55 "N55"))
  (pad 4 smd rect (at 1.165 0.95 90) (size 0.58 1.39) (layers F.Cu F.Paste F.Mask) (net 53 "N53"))
  (pad 5 smd rect (at 1.165 -0.95 90) (size 0.58 1.39) (layers F.Cu F.Paste F.Mask) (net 3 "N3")))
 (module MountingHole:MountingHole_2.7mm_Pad (layer F.Cu) (at 138.5 108.5 180)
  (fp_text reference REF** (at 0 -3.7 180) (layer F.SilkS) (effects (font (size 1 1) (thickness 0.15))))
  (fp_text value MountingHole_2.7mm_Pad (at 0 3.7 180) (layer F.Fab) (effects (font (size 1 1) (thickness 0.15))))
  (pad 1 thru_hole circle (at 0 0 180) (size 6 6) (drill 2.7) (layers *.Cu *.Mask)))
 (gr_line (start 135 47) (end 191 47) (layer Edge.Cuts) (width 0.15))
 (gr_line (start 135 112) (end 135 47) (layer Edge.Cuts) (width 0.15))
 (gr_line (start 191 112) (end 135 112) (layer Edge.Cuts) (width 0.15))
 (gr_line (start 191 47) (end 191 112) (layer Edge.Cuts) (width 0.15))
 (segment (start 159.5025 52) (end 158.44 53.0625) (width 0.25) (layer F.Cu) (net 1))
 (segment (start 162.05 52) (end 159.5025 52) (width 0.25) (layer F.Cu) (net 1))
 (segment (start 164.6 52) (end 163.95 52) (width 0.25) (layer F.Cu) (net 2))
 (segment (start 176.177919 52) (end 164.6 52) (width 0.25) (layer F.Cu) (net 2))
 (segment (start 184.757919 60.58) (end 176.177919 52) (width 0.25) (layer F.Cu) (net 2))
 (segment (start 185.96 60.58) (end 184.757919 60.58) (width 0.25) (layer F.Cu) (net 2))
 (via (at 156.5 61.5) (size 0.8) (drill 0.4) (layers F.Cu B.Cu) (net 4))
 (via (at 156.5 56) (size 0.8) (drill 0.4) (layers F.Cu B.Cu) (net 4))
 (segment (start 156.5 56) (end 156.5 61.5) (width 0.25) (layer B.Cu) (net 4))
 (segment (start 157.3775 56) (end 158.44 54.9375) (width 0.25) (layer F.Cu) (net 4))
 (segment (start 156.5 56) (end 157.3775 56) (width 0.25) (layer F.Cu) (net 4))
 (segment (start 157.97 61.5) (end 158.28 61.19) (width 0.25) (layer F.Cu) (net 4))
 (segment (start 156.5 61.5) (end 157.97 61.5) (width 0.25) (layer F.Cu) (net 4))
 (segment (start 154.0875 58.65) (end 154 58.5625) (width 0.25) (layer F.Cu) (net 5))
 (segment (start 158.28 58.65) (end 154.0875 58.65) (width 0.25) (layer F.Cu) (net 5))
 (segment (start 150.5 60.5) (end 152.4375 58.5625) (width 0.25) (layer F.Cu) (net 5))
 (segment (start 152.4375 58.5625) (end 154 58.5625) (width 0.25) (layer F.Cu) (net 5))
 (segment (start 148.7875 60.5) (end 150.5 60.5) (width 0.25) (layer F.Cu) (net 5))
 (segment (start 150.5 65.7875) (end 148.7875 67.5) (width 0.25) (layer F.Cu) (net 5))
 (segment (start 150.5 62.2125) (end 150.5 65.7875) (width 0.25) (layer F.Cu) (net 5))
 (segment (start 148.7875 60.5) (end 150.5 62.2125) (width 0.25) (layer F.Cu) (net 5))
 (segment (start 155.2175 73.93) (end 155.2175 74.16) (width 0.25) (layer F.Cu) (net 5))
 (segment (start 148.7875 67.5) (end 155.2175 73.93) (width 0.25) (layer F.Cu) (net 5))
 (segment (start 155.2175 74.735) (end 157 76.5175) (width 0.25) (layer F.Cu) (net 5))
 (segment (start 155.2175 74.16) (end 155.2175 74.735) (width 0.25) (layer F.Cu) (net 5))
 (segment (start 157 79.9975) (end 155.2175 81.78) (width 0.25) (layer F.Cu) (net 5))
 (segment (start 157 76.5175) (end 157 79.9975) (width 0.25) (layer F.Cu) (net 5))
 (segment (start 150.2175 85.7825) (end 150.2175 88.4) (width 0.25) (layer F.Cu) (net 5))
 (segment (start 155.2175 81.78) (end 155.2175 82.355) (width 0.25) (layer F.Cu) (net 5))
 (segment (start 153.5725 84) (end 152 84) (width 0.25) (layer F.Cu) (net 5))
 (segment (start 155.2175 82.355) (end 153.5725 84) (width 0.25) (layer F.Cu) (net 5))
 (segment (start 152 84) (end 150.2175 85.7825) (width 0.25) (layer F.Cu) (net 5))
 (segment (start 150.2175 88.975) (end 151.2425 90) (width 0.25) (layer F.Cu) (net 5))
 (segment (start 150.2175 88.4) (end 150.2175 88.975) (width 0.25) (layer F.Cu) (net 5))
 (segment (start 151.2425 90) (end 152 90) (width 0.25) (layer F.Cu) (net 5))
 (segment (start 152 90) (end 152.5 90.5) (width 0.25) (layer F.Cu) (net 5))
 (segment (start 152.5 93.2175) (end 150.2175 95.5) (width 0.25) (layer F.Cu) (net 5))
 (segment (start 152.5 90.5) (end 152.5 93.2175) (width 0.25) (layer F.Cu) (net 5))
 (segment (start 150.2175 95.5) (end 152 97.2825) (width 0.25) (layer F.Cu) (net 5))
 (segment (start 152 97.2825) (end 152 101.5) (width 0.25) (layer F.Cu) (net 5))
 (segment (start 151.2875 101.5) (end 150.2875 102.5) (width 0.25) (layer F.Cu) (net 5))
 (segment (start 152 101.5) (end 151.2875 101.5) (width 0.25) (layer F.Cu) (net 5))
 (segment (start 154 60.4375) (end 155.5625 60.4375) (width 0.25) (layer F.Cu) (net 6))
 (segment (start 156.08 59.92) (end 158.28 59.92) (width 0.25) (layer F.Cu) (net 6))
 (segment (start 155.5625 60.4375) (end 156.08 59.92) (width 0.25) (layer F.Cu) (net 6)))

